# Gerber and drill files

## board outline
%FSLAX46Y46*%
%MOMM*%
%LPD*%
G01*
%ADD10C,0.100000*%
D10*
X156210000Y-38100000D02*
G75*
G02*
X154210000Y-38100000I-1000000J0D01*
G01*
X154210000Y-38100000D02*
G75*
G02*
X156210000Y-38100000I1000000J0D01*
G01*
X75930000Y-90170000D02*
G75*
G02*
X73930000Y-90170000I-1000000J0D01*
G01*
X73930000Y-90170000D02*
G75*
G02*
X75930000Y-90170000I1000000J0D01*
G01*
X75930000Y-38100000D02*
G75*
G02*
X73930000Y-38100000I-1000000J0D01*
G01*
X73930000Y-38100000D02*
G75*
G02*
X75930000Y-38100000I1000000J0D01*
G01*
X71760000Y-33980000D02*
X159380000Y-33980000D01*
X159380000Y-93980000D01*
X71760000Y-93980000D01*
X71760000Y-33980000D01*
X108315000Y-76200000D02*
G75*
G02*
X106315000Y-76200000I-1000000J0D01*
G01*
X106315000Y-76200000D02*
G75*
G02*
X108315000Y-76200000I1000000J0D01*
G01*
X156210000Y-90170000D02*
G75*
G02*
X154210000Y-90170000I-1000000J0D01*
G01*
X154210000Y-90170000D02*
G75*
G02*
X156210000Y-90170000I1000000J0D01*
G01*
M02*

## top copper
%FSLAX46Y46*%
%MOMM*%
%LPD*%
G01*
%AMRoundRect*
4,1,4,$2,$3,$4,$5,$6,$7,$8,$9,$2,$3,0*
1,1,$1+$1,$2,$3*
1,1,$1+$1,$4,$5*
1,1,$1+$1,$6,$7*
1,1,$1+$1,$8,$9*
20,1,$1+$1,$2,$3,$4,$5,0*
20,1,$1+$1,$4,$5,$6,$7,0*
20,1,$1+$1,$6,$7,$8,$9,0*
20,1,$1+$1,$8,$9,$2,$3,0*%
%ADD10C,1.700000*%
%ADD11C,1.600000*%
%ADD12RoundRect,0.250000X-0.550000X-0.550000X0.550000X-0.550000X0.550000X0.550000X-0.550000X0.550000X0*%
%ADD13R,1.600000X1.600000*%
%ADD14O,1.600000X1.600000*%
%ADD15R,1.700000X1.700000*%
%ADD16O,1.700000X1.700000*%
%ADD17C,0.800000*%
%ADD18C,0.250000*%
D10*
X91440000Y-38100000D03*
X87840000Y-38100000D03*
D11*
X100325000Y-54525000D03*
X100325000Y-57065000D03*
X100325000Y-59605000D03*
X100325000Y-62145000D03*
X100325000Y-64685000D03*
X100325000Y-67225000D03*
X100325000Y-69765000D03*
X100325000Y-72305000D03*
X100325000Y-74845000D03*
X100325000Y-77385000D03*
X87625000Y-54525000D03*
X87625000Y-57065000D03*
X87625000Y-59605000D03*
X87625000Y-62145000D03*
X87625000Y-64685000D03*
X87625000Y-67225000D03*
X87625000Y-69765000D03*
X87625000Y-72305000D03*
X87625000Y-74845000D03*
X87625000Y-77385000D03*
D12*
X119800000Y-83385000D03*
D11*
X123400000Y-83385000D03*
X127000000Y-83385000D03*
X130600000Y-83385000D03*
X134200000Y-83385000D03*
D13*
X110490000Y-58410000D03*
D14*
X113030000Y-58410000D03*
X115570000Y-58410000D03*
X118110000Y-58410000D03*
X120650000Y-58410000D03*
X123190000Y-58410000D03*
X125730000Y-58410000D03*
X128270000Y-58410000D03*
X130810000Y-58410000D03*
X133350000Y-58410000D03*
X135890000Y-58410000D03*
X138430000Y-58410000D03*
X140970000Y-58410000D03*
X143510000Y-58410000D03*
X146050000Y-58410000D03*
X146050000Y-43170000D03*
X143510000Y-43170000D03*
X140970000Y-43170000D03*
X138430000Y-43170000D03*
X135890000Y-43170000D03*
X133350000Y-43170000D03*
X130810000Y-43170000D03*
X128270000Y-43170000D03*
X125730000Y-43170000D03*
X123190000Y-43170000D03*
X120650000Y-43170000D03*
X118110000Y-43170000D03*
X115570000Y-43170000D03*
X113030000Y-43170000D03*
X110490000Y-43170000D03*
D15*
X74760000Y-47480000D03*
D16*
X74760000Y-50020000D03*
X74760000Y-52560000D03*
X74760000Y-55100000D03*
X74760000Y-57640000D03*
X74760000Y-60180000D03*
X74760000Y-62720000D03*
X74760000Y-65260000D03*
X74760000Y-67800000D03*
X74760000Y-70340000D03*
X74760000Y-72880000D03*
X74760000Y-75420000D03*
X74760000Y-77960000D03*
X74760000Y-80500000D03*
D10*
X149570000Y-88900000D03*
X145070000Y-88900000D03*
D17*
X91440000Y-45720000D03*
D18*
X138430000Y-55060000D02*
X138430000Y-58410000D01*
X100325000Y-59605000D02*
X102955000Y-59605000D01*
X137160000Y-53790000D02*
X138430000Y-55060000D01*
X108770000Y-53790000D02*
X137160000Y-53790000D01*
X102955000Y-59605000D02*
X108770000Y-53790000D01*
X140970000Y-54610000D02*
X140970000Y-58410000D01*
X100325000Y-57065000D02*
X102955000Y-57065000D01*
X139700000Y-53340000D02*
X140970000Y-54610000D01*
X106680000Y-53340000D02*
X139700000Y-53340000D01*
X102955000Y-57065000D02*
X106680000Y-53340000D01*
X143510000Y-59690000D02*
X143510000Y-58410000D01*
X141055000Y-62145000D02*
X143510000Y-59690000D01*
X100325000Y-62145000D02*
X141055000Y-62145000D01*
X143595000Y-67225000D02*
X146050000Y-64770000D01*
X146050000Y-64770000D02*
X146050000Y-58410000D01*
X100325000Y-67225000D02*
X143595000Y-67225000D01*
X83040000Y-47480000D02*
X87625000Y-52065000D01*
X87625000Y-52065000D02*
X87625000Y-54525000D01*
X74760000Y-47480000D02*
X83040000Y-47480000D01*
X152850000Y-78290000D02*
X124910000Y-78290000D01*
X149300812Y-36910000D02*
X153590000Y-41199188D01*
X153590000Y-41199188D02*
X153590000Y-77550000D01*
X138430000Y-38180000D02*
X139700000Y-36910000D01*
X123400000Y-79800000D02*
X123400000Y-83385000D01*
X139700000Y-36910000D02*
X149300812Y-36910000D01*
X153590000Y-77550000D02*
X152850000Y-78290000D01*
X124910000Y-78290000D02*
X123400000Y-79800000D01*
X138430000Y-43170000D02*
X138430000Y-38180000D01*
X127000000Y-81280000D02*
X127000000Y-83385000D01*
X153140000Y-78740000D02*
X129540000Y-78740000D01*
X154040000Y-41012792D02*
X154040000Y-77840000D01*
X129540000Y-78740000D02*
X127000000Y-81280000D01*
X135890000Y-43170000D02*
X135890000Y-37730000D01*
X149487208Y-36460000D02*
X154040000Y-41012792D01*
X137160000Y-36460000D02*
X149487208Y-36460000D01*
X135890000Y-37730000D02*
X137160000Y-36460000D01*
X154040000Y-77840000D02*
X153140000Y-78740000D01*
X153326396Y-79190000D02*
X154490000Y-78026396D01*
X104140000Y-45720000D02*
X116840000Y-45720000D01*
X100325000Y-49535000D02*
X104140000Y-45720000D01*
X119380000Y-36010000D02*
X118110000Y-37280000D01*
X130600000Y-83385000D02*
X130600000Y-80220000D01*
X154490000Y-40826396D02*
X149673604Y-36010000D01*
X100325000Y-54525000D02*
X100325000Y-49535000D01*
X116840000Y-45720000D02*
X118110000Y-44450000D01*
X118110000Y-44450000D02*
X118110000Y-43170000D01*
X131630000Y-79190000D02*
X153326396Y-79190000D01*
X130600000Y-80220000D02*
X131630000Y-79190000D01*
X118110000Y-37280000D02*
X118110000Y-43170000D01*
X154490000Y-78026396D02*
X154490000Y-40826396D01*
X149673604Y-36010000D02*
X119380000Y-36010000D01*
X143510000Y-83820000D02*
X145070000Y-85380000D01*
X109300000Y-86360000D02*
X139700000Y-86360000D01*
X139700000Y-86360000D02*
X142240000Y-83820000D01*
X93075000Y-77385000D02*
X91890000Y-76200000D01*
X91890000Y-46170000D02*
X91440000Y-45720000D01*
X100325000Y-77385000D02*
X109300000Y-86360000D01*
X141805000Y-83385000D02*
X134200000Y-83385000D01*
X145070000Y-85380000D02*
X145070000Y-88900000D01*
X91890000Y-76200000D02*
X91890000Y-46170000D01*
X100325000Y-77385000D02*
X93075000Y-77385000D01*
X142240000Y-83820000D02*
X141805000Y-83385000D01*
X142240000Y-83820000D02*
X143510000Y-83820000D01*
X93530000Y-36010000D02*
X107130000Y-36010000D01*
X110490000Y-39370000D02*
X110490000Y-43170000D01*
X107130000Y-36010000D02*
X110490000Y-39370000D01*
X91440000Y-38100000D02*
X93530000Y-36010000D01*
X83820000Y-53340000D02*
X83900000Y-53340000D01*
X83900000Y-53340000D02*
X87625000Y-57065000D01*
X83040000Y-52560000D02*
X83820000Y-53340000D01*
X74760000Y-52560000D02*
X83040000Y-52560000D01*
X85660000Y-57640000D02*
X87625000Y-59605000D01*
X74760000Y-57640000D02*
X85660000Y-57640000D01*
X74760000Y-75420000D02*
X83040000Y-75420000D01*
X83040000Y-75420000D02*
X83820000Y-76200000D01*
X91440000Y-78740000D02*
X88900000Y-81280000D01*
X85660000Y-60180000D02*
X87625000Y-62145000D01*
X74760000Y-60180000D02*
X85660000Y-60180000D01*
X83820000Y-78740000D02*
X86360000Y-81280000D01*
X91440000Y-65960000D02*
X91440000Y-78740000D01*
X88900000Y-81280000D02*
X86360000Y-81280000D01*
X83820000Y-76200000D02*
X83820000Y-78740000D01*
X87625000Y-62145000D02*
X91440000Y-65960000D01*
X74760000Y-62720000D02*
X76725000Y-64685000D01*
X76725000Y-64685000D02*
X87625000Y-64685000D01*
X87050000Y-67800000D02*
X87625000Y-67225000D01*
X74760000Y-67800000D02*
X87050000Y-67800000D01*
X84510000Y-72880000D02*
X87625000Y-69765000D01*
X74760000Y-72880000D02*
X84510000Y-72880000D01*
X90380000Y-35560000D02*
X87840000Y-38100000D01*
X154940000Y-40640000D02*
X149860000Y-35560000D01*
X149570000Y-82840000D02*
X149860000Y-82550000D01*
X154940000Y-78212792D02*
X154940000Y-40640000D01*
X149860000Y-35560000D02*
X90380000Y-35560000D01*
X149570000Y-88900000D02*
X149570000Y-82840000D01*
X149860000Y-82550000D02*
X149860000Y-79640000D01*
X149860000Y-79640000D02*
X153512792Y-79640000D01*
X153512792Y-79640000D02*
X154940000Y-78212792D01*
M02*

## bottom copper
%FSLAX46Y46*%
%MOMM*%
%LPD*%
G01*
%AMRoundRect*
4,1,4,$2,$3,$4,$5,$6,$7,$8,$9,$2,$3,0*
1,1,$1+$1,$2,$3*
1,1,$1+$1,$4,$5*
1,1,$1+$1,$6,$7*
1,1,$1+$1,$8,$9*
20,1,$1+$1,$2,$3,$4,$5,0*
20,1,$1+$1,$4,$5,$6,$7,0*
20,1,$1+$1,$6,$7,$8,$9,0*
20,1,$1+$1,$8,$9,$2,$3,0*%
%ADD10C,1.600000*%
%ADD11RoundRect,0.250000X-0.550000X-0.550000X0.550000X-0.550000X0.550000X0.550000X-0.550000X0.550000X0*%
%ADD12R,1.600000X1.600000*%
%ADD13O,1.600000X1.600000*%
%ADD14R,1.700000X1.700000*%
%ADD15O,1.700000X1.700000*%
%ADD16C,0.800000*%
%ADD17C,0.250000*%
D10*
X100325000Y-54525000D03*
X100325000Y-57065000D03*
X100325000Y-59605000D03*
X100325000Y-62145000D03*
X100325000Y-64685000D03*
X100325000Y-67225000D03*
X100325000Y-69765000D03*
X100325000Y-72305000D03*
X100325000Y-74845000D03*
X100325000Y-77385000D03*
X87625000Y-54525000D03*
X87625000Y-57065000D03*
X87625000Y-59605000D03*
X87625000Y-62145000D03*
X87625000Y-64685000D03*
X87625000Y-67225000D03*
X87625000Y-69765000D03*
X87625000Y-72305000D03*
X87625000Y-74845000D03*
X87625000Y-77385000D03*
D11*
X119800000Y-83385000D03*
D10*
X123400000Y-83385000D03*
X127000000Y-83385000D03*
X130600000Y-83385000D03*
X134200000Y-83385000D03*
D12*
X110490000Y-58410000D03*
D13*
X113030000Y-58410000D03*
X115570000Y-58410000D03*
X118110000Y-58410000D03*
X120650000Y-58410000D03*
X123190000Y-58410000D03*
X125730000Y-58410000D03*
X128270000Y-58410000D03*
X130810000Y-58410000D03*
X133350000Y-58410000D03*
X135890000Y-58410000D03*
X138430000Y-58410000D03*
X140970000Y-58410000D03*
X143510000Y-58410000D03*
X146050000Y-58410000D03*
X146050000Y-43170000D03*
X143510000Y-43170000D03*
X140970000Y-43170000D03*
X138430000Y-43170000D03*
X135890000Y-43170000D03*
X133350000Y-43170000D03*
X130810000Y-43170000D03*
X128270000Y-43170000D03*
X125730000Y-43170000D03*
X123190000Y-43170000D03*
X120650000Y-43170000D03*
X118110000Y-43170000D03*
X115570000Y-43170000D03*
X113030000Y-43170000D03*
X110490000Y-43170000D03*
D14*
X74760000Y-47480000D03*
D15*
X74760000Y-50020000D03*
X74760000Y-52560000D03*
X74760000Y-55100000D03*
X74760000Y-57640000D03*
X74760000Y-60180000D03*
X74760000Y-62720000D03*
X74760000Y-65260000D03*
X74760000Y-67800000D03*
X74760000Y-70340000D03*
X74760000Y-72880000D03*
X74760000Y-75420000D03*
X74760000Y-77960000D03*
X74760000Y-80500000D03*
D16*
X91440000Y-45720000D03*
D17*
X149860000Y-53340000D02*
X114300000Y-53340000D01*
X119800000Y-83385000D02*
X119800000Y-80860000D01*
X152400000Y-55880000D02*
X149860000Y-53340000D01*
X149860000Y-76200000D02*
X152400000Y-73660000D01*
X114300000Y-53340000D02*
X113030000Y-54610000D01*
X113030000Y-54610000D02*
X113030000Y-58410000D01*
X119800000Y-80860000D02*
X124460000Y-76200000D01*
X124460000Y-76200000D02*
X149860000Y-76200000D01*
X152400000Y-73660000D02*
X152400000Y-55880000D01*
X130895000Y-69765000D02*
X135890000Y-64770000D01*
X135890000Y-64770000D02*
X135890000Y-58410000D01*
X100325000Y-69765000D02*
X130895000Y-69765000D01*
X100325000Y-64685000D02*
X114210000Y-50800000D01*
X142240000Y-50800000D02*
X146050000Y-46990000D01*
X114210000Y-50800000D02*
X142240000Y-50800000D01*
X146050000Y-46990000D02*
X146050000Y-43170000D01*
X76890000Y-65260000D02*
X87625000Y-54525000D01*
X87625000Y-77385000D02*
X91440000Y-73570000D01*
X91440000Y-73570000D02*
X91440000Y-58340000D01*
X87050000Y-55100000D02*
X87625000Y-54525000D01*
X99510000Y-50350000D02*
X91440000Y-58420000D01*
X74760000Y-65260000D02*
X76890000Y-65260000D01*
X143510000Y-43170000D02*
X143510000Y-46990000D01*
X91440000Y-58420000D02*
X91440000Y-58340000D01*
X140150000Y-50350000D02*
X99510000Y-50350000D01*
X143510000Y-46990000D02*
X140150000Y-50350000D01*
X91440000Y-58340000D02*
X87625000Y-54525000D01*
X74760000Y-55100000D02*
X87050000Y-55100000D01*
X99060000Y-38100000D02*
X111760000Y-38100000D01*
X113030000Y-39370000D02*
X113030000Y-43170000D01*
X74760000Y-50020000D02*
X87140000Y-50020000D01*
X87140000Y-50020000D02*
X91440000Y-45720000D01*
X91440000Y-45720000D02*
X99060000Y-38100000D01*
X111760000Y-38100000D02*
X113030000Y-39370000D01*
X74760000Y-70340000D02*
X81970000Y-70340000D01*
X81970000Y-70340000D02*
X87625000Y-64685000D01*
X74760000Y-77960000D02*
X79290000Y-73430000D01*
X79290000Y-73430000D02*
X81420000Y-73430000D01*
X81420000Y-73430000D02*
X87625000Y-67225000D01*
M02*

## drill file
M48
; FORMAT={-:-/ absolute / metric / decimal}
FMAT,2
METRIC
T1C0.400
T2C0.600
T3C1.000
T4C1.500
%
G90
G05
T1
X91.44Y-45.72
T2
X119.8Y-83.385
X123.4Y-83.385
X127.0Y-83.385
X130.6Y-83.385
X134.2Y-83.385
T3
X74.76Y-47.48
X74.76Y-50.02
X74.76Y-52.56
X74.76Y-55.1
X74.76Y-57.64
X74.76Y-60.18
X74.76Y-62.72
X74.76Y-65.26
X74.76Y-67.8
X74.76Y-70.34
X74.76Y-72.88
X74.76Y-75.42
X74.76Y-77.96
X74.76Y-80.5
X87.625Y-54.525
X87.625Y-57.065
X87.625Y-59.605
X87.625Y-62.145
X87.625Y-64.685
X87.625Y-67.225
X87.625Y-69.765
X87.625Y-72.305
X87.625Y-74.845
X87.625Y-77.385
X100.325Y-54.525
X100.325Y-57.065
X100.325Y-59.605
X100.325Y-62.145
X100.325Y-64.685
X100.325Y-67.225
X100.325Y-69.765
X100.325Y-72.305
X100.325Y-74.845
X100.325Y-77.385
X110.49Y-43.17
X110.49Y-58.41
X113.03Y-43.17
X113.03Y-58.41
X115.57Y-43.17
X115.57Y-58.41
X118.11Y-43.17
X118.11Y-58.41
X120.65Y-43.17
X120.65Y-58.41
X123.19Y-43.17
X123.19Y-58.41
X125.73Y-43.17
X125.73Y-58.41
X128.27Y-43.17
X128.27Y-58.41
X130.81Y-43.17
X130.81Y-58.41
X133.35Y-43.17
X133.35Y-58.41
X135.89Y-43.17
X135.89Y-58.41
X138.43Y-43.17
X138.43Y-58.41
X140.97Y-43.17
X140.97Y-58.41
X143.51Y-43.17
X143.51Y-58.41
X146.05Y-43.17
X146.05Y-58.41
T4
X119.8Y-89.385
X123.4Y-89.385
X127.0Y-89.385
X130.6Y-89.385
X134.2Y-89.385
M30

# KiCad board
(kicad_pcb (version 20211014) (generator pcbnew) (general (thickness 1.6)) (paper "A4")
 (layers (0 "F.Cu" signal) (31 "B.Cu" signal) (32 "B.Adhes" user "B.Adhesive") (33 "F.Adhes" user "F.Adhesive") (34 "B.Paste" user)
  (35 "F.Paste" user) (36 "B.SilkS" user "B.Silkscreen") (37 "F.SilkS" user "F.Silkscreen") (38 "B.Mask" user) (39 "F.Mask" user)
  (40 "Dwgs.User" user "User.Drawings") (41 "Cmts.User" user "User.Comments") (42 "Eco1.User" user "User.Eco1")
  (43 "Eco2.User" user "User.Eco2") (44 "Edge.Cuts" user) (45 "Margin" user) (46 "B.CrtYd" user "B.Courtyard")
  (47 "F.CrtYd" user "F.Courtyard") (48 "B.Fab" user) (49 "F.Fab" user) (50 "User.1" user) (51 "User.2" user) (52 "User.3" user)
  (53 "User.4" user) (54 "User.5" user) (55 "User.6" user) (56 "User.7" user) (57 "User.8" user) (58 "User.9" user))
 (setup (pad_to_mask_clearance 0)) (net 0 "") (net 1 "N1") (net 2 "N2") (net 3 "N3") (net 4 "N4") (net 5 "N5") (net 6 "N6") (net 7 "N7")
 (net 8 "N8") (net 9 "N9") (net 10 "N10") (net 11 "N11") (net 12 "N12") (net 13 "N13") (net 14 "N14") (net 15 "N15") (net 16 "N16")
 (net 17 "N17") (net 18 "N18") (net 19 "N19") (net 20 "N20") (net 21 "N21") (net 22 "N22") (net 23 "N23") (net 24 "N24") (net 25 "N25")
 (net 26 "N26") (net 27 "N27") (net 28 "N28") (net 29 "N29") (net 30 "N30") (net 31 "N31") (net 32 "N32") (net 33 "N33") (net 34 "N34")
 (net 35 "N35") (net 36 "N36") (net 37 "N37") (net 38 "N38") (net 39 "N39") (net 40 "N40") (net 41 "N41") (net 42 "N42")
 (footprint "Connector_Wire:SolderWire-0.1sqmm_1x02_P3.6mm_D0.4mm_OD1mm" (layer "F.Cu") (at 91.44 38.1 180)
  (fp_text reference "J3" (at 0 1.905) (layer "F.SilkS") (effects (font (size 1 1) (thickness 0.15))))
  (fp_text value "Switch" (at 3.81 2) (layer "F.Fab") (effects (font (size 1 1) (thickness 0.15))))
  (pad "1" smd circle (at 0 0 180) (size 1.7 1.7) (layers "F.Cu" "F.Paste" "F.Mask") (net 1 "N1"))
  (pad "2" smd circle (at 3.6 0 180) (size 1.7 1.7) (layers "F.Cu" "F.Paste" "F.Mask") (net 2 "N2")))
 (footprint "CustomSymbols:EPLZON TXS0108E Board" (layer "F.Cu") (at 101.595 53.255 -90)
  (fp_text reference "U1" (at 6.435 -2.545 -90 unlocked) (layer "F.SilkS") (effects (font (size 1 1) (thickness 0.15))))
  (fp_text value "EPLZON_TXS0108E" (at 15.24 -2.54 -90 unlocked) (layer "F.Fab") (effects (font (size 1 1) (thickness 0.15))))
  (pad "1" thru_hole circle (at 1.27 1.27 270) (size 1.6 1.6) (drill 1) (layers *.Cu *.Mask) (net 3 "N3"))
  (pad "2" thru_hole circle (at 3.81 1.27 270) (size 1.6 1.6) (drill 1) (layers *.Cu *.Mask) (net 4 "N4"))
  (pad "3" thru_hole circle (at 6.35 1.27 270) (size 1.6 1.6) (drill 1) (layers *.Cu *.Mask) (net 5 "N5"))
  (pad "4" thru_hole circle (at 8.89 1.27 270) (size 1.6 1.6) (drill 1) (layers *.Cu *.Mask) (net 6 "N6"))
  (pad "5" thru_hole circle (at 11.43 1.27 270) (size 1.6 1.6) (drill 1) (layers *.Cu *.Mask) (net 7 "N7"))
  (pad "6" thru_hole circle (at 13.97 1.27 270) (size 1.6 1.6) (drill 1) (layers *.Cu *.Mask) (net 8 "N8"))
  (pad "7" thru_hole circle (at 16.51 1.27 270) (size 1.6 1.6) (drill 1) (layers *.Cu *.Mask) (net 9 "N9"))
  (pad "8" thru_hole circle (at 19.05 1.27 270) (size 1.6 1.6) (drill 1) (layers *.Cu *.Mask) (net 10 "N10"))
  (pad "9" thru_hole circle (at 21.59 1.27 270) (size 1.6 1.6) (drill 1) (layers *.Cu *.Mask) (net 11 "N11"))
  (pad "10" thru_hole circle (at 24.13 1.27 270) (size 1.6 1.6) (drill 1) (layers *.Cu *.Mask) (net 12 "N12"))
  (pad "11" thru_hole circle (at 1.27 13.97 270) (size 1.6 1.6) (drill 1) (layers *.Cu *.Mask) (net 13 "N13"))
  (pad "12" thru_hole circle (at 3.81 13.97 270) (size 1.6 1.6) (drill 1) (layers *.Cu *.Mask) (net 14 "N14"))
  (pad "13" thru_hole circle (at 6.35 13.97 270) (size 1.6 1.6) (drill 1) (layers *.Cu *.Mask) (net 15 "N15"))
  (pad "14" thru_hole circle (at 8.89 13.97 270) (size 1.6 1.6) (drill 1) (layers *.Cu *.Mask) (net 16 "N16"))
  (pad "15" thru_hole circle (at 11.43 13.97 270) (size 1.6 1.6) (drill 1) (layers *.Cu *.Mask) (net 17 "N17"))
  (pad "16" thru_hole circle (at 13.97 13.97 270) (size 1.6 1.6) (drill 1) (layers *.Cu *.Mask) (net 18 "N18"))
  (pad "17" thru_hole circle (at 16.51 13.97 270) (size 1.6 1.6) (drill 1) (layers *.Cu *.Mask) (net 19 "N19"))
  (pad "18" thru_hole circle (at 19.05 13.97 270) (size 1.6 1.6) (drill 1) (layers *.Cu *.Mask) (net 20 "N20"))
  (pad "19" thru_hole circle (at 21.59 13.97 270) (size 1.6 1.6) (drill 1) (layers *.Cu *.Mask) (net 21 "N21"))
  (pad "20" thru_hole circle (at 24.13 13.97 270) (size 1.6 1.6) (drill 1) (layers *.Cu *.Mask) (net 13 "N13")))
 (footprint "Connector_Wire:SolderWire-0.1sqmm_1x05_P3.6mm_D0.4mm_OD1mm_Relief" (layer "F.Cu") (at 119.8 83.385)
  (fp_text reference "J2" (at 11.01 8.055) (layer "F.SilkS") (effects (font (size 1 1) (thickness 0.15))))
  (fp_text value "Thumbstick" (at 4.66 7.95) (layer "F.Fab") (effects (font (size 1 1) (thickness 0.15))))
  (pad "" np_thru_hole circle (at 10.8 6) (size 1.5 1.5) (drill 1.5) (layers *.Cu *.Mask))
  (pad "" np_thru_hole circle (at 3.6 6) (size 1.5 1.5) (drill 1.5) (layers *.Cu *.Mask))
  (pad "" np_thru_hole circle (at 0 6) (size 1.5 1.5) (drill 1.5) (layers *.Cu *.Mask))
  (pad "" np_thru_hole circle (at 14.4 6) (size 1.5 1.5) (drill 1.5) (layers *.Cu *.Mask))
  (pad "" np_thru_hole circle (at 7.2 6) (size 1.5 1.5) (drill 1.5) (layers *.Cu *.Mask))
  (pad "1" thru_hole roundrect (at 0 0) (size 1.6 1.6) (drill 0.6) (layers *.Cu *.Mask) (roundrect_rratio 0.15625) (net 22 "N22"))
  (pad "2" thru_hole circle (at 3.6 0) (size 1.6 1.6) (drill 0.6) (layers *.Cu *.Mask) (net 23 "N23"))
  (pad "3" thru_hole circle (at 7.2 0) (size 1.6 1.6) (drill 0.6) (layers *.Cu *.Mask) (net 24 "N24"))
  (pad "4" thru_hole circle (at 10.8 0) (size 1.6 1.6) (drill 0.6) (layers *.Cu *.Mask) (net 3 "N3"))
  (pad "5" thru_hole circle (at 14.4 0) (size 1.6 1.6) (drill 0.6) (layers *.Cu *.Mask) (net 12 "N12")))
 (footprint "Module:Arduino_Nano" (layer "F.Cu") (at 110.49 58.41 90)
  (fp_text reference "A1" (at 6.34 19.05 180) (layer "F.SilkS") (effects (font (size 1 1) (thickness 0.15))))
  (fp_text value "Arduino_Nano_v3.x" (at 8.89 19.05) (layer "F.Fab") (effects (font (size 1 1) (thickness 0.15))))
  (pad "1" thru_hole rect (at 0 0 90) (size 1.6 1.6) (drill 1) (layers *.Cu *.Mask) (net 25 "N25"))
  (pad "2" thru_hole oval (at 0 2.54 90) (size 1.6 1.6) (drill 1) (layers *.Cu *.Mask) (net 22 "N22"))
  (pad "3" thru_hole oval (at 0 5.08 90) (size 1.6 1.6) (drill 1) (layers *.Cu *.Mask) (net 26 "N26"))
  (pad "4" thru_hole oval (at 0 7.62 90) (size 1.6 1.6) (drill 1) (layers *.Cu *.Mask) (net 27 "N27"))
  (pad "5" thru_hole oval (at 0 10.16 90) (size 1.6 1.6) (drill 1) (layers *.Cu *.Mask) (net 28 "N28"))
  (pad "6" thru_hole oval (at 0 12.7 90) (size 1.6 1.6) (drill 1) (layers *.Cu *.Mask) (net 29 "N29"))
  (pad "7" thru_hole oval (at 0 15.24 90) (size 1.6 1.6) (drill 1) (layers *.Cu *.Mask) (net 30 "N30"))
  (pad "8" thru_hole oval (at 0 17.78 90) (size 1.6 1.6) (drill 1) (layers *.Cu *.Mask) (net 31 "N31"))
  (pad "9" thru_hole oval (at 0 20.32 90) (size 1.6 1.6) (drill 1) (layers *.Cu *.Mask) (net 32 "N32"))
  (pad "10" thru_hole oval (at 0 22.86 90) (size 1.6 1.6) (drill 1) (layers *.Cu *.Mask) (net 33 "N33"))
  (pad "11" thru_hole oval (at 0 25.4 90) (size 1.6 1.6) (drill 1) (layers *.Cu *.Mask) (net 9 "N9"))
  (pad "12" thru_hole oval (at 0 27.94 90) (size 1.6 1.6) (drill 1) (layers *.Cu *.Mask) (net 5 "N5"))
  (pad "13" thru_hole oval (at 0 30.48 90) (size 1.6 1.6) (drill 1) (layers *.Cu *.Mask) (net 4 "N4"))
  (pad "14" thru_hole oval (at 0 33.02 90) (size 1.6 1.6) (drill 1) (layers *.Cu *.Mask) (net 6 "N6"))
  (pad "15" thru_hole oval (at 0 35.56 90) (size 1.6 1.6) (drill 1) (layers *.Cu *.Mask) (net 8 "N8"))
  (pad "16" thru_hole oval (at 15.24 35.56 90) (size 1.6 1.6) (drill 1) (layers *.Cu *.Mask) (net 7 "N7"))
  (pad "17" thru_hole oval (at 15.24 33.02 90) (size 1.6 1.6) (drill 1) (layers *.Cu *.Mask) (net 13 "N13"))
  (pad "18" thru_hole oval (at 15.24 30.48 90) (size 1.6 1.6) (drill 1) (layers *.Cu *.Mask) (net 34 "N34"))
  (pad "19" thru_hole oval (at 15.24 27.94 90) (size 1.6 1.6) (drill 1) (layers *.Cu *.Mask) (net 23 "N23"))
  (pad "20" thru_hole oval (at 15.24 25.4 90) (size 1.6 1.6) (drill 1) (layers *.Cu *.Mask) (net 24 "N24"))
  (pad "21" thru_hole oval (at 15.24 22.86 90) (size 1.6 1.6) (drill 1) (layers *.Cu *.Mask) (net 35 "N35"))
  (pad "22" thru_hole oval (at 15.24 20.32 90) (size 1.6 1.6) (drill 1) (layers *.Cu *.Mask) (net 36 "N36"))
  (pad "23" thru_hole oval (at 15.24 17.78 90) (size 1.6 1.6) (drill 1) (layers *.Cu *.Mask) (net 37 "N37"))
  (pad "24" thru_hole oval (at 15.24 15.24 90) (size 1.6 1.6) (drill 1) (layers *.Cu *.Mask) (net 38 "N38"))
  (pad "25" thru_hole oval (at 15.24 12.7 90) (size 1.6 1.6) (drill 1) (layers *.Cu *.Mask) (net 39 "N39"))
  (pad "26" thru_hole oval (at 15.24 10.16 90) (size 1.6 1.6) (drill 1) (layers *.Cu *.Mask) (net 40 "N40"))
  (pad "27" thru_hole oval (at 15.24 7.62 90) (size 1.6 1.6) (drill 1) (layers *.Cu *.Mask) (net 3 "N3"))
  (pad "28" thru_hole oval (at 15.24 5.08 90) (size 1.6 1.6) (drill 1) (layers *.Cu *.Mask) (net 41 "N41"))
  (pad "29" thru_hole oval (at 15.24 2.54 90) (size 1.6 1.6) (drill 1) (layers *.Cu *.Mask) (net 12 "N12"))
  (pad "30" thru_hole oval (at 15.24 0 90) (size 1.6 1.6) (drill 1) (layers *.Cu *.Mask) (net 1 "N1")))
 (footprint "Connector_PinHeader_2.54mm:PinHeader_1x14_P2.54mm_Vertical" (layer "F.Cu") (at 74.76 47.48)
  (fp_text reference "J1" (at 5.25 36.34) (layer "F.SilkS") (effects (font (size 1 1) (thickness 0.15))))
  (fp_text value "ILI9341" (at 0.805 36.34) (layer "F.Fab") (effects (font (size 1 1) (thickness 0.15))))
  (pad "1" thru_hole rect (at 0 0) (size 1.7 1.7) (drill 1) (layers *.Cu *.Mask) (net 13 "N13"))
  (pad "2" thru_hole oval (at 0 2.54) (size 1.7 1.7) (drill 1) (layers *.Cu *.Mask) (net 12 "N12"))
  (pad "3" thru_hole oval (at 0 5.08) (size 1.7 1.7) (drill 1) (layers *.Cu *.Mask) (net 14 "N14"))
  (pad "4" thru_hole oval (at 0 7.62) (size 1.7 1.7) (drill 1) (layers *.Cu *.Mask) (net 13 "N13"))
  (pad "5" thru_hole oval (at 0 10.16) (size 1.7 1.7) (drill 1) (layers *.Cu *.Mask) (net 15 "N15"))
  (pad "6" thru_hole oval (at 0 12.7) (size 1.7 1.7) (drill 1) (layers *.Cu *.Mask) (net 16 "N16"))
  (pad "7" thru_hole oval (at 0 15.24) (size 1.7 1.7) (drill 1) (layers *.Cu *.Mask) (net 17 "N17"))
  (pad "8" thru_hole oval (at 0 17.78) (size 1.7 1.7) (drill 1) (layers *.Cu *.Mask) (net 13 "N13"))
  (pad "9" thru_hole oval (at 0 20.32) (size 1.7 1.7) (drill 1) (layers *.Cu *.Mask) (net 18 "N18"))
  (pad "10" thru_hole oval (at 0 22.86) (size 1.7 1.7) (drill 1) (layers *.Cu *.Mask) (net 17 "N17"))
  (pad "11" thru_hole oval (at 0 25.4) (size 1.7 1.7) (drill 1) (layers *.Cu *.Mask) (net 19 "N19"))
  (pad "12" thru_hole oval (at 0 27.94) (size 1.7 1.7) (drill 1) (layers *.Cu *.Mask) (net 16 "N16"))
  (pad "13" thru_hole oval (at 0 30.48) (size 1.7 1.7) (drill 1) (layers *.Cu *.Mask) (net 18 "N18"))
  (pad "14" thru_hole oval (at 0 33.02) (size 1.7 1.7) (drill 1) (layers *.Cu *.Mask) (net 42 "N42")))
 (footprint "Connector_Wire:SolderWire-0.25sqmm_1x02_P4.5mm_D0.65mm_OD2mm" (layer "F.Cu") (at 149.57 88.9 180)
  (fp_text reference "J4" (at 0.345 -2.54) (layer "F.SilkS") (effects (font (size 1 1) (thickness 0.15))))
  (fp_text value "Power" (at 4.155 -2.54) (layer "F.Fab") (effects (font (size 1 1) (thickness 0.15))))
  (pad "1" smd circle (at 0 0 180) (size 1.7 1.7) (layers "F.Cu" "F.Paste" "F.Mask") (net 2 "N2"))
  (pad "2" smd circle (at 4.5 0 180) (size 1.7 1.7) (layers "F.Cu" "F.Paste" "F.Mask") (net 12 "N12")))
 (gr_circle (center 155.21 38.1) (end 156.21 38.1) (layer "Edge.Cuts") (width 0.1) (fill none))
 (gr_circle (center 74.93 90.17) (end 75.93 90.17) (layer "Edge.Cuts") (width 0.1) (fill none))
 (gr_circle (center 74.93 38.1) (end 75.93 38.1) (layer "Edge.Cuts") (width 0.1) (fill none))
 (gr_rect (start 71.76 33.98) (end 159.38 93.98) (layer "Edge.Cuts") (width 0.1) (fill none))
 (gr_circle (center 107.315 76.2) (end 108.315 76.2) (layer "Edge.Cuts") (width 0.1) (fill none))
 (gr_circle (center 155.21 90.17) (end 156.21 90.17) (layer "Edge.Cuts") (width 0.1) (fill none))
 (segment (start 149.86 53.34) (end 114.3 53.34) (width 0.25) (layer "B.Cu") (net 22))
 (segment (start 119.8 83.385) (end 119.8 80.86) (width 0.25) (layer "B.Cu") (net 22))
 (segment (start 152.4 55.88) (end 149.86 53.34) (width 0.25) (layer "B.Cu") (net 22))
 (segment (start 149.86 76.2) (end 152.4 73.66) (width 0.25) (layer "B.Cu") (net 22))
 (segment (start 114.3 53.34) (end 113.03 54.61) (width 0.25) (layer "B.Cu") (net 22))
 (segment (start 113.03 54.61) (end 113.03 58.41) (width 0.25) (layer "B.Cu") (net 22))
 (segment (start 119.8 80.86) (end 124.46 76.2) (width 0.25) (layer "B.Cu") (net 22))
 (segment (start 124.46 76.2) (end 149.86 76.2) (width 0.25) (layer "B.Cu") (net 22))
 (segment (start 152.4 73.66) (end 152.4 55.88) (width 0.25) (layer "B.Cu") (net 22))
 (segment (start 130.895 69.765) (end 135.89 64.77) (width 0.25) (layer "B.Cu") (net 9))
 (segment (start 135.89 64.77) (end 135.89 58.41) (width 0.25) (layer "B.Cu") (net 9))
 (segment (start 100.325 69.765) (end 130.895 69.765) (width 0.25) (layer "B.Cu") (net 9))
 (segment (start 138.43 55.06) (end 138.43 58.41) (width 0.25) (layer "F.Cu") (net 5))
 (segment (start 100.325 59.605) (end 102.955 59.605) (width 0.25) (layer "F.Cu") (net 5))
 (segment (start 137.16 53.79) (end 138.43 55.06) (width 0.25) (layer "F.Cu") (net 5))
 (segment (start 108.77 53.79) (end 137.16 53.79) (width 0.25) (layer "F.Cu") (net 5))
 (segment (start 102.955 59.605) (end 108.77 53.79) (width 0.25) (layer "F.Cu") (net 5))
 (segment (start 140.97 54.61) (end 140.97 58.41) (width 0.25) (layer "F.Cu") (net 4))
 (segment (start 100.325 57.065) (end 102.955 57.065) (width 0.25) (layer "F.Cu") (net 4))
 (segment (start 139.7 53.34) (end 140.97 54.61) (width 0.25) (layer "F.Cu") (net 4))
 (segment (start 106.68 53.34) (end 139.7 53.34) (width 0.25) (layer "F.Cu") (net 4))
 (segment (start 102.955 57.065) (end 106.68 53.34) (width 0.25) (layer "F.Cu") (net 4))
 (segment (start 143.51 59.69) (end 143.51 58.41) (width 0.25) (layer "F.Cu") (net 6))
 (segment (start 141.055 62.145) (end 143.51 59.69) (width 0.25) (layer "F.Cu") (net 6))
 (segment (start 100.325 62.145) (end 141.055 62.145) (width 0.25) (layer "F.Cu") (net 6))
 (segment (start 143.595 67.225) (end 146.05 64.77) (width 0.25) (layer "F.Cu") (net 8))
 (segment (start 146.05 64.77) (end 146.05 58.41) (width 0.25) (layer "F.Cu") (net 8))
 (segment (start 100.325 67.225) (end 143.595 67.225) (width 0.25) (layer "F.Cu") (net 8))
 (segment (start 100.325 64.685) (end 114.21 50.8) (width 0.25) (layer "B.Cu") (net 7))
 (segment (start 142.24 50.8) (end 146.05 46.99) (width 0.25) (layer "B.Cu") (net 7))
 (segment (start 114.21 50.8) (end 142.24 50.8) (width 0.25) (layer "B.Cu") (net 7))
 (segment (start 146.05 46.99) (end 146.05 43.17) (width 0.25) (layer "B.Cu") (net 7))
 (segment (start 83.04 47.48) (end 87.625 52.065) (width 0.25) (layer "F.Cu") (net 13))
 (segment (start 87.625 52.065) (end 87.625 54.525) (width 0.25) (layer "F.Cu") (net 13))
 (segment (start 74.76 47.48) (end 83.04 47.48) (width 0.25) (layer "F.Cu") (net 13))
 (segment (start 76.89 65.26) (end 87.625 54.525) (width 0.25) (layer "B.Cu") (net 13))
 (segment (start 87.625 77.385) (end 91.44 73.57) (width 0.25) (layer "B.Cu") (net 13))
 (segment (start 91.44 73.57) (end 91.44 58.34) (width 0.25) (layer "B.Cu") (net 13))
 (segment (start 87.05 55.1) (end 87.625 54.525) (width 0.25) (layer "B.Cu") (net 13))
 (segment (start 99.51 50.35) (end 91.44 58.42) (width 0.25) (layer "B.Cu") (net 13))
 (segment (start 74.76 65.26) (end 76.89 65.26) (width 0.25) (layer "B.Cu") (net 13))
 (segment (start 143.51 43.17) (end 143.51 46.99) (width 0.25) (layer "B.Cu") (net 13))
 (segment (start 91.44 58.42) (end 91.44 58.34) (width 0.25) (layer "B.Cu") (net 13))
 (segment (start 140.15 50.35) (end 99.51 50.35) (width 0.25) (layer "B.Cu") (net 13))
 (segment (start 143.51 46.99) (end 140.15 50.35) (width 0.25) (layer "B.Cu") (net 13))
 (segment (start 91.44 58.34) (end 87.625 54.525) (width 0.25) (layer "B.Cu") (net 13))
 (segment (start 74.76 55.1) (end 87.05 55.1) (width 0.25) (layer "B.Cu") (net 13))
 (segment (start 152.85 78.29) (end 124.91 78.29) (width 0.25) (layer "F.Cu") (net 23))
 (segment (start 149.300812 36.91) (end 153.59 41.199188) (width 0.25) (layer "F.Cu") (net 23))
 (segment (start 153.59 41.199188) (end 153.59 77.55) (width 0.25) (layer "F.Cu") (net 23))
 (segment (start 138.43 38.18) (end 139.7 36.91) (width 0.25) (layer "F.Cu") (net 23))
 (segment (start 123.4 79.8) (end 123.4 83.385) (width 0.25) (layer "F.Cu") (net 23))
 (segment (start 139.7 36.91) (end 149.300812 36.91) (width 0.25) (layer "F.Cu") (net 23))
 (segment (start 153.59 77.55) (end 152.85 78.29) (width 0.25) (layer "F.Cu") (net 23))
 (segment (start 124.91 78.29) (end 123.4 79.8) (width 0.25) (layer "F.Cu") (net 23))
 (segment (start 138.43 43.17) (end 138.43 38.18) (width 0.25) (layer "F.Cu") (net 23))
 (segment (start 127 81.28) (end 127 83.385) (width 0.25) (layer "F.Cu") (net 24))
 (segment (start 153.14 78.74) (end 129.54 78.74) (width 0.25) (layer "F.Cu") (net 24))
 (segment (start 154.04 41.012792) (end 154.04 77.84) (width 0.25) (layer "F.Cu") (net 24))
 (segment (start 129.54 78.74) (end 127 81.28) (width 0.25) (layer "F.Cu") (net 24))
 (segment (start 135.89 43.17) (end 135.89 37.73) (width 0.25) (layer "F.Cu") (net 24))
 (segment (start 149.487208 36.46) (end 154.04 41.012792) (width 0.25) (layer "F.Cu") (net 24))
 (segment (start 137.16 36.46) (end 149.487208 36.46) (width 0.25) (layer "F.Cu") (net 24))
 (segment (start 135.89 37.73) (end 137.16 36.46) (width 0.25) (layer "F.Cu") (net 24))
 (segment (start 154.04 77.84) (end 153.14 78.74) (width 0.25) (layer "F.Cu") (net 24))
 (segment (start 153.326396 79.19) (end 154.49 78.026396) (width 0.25) (layer "F.Cu") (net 3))
 (segment (start 104.14 45.72) (end 116.84 45.72) (width 0.25) (layer "F.Cu") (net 3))
 (segment (start 100.325 49.535) (end 104.14 45.72) (width 0.25) (layer "F.Cu") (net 3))
 (segment (start 119.38 36.01) (end 118.11 37.28) (width 0.25) (layer "F.Cu") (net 3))
 (segment (start 130.6 83.385) (end 130.6 80.22) (width 0.25) (layer "F.Cu") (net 3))
 (segment (start 154.49 40.826396) (end 149.673604 36.01) (width 0.25) (layer "F.Cu") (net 3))
 (segment (start 100.325 54.525) (end 100.325 49.535) (width 0.25) (layer "F.Cu") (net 3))
 (segment (start 116.84 45.72) (end 118.11 44.45) (width 0.25) (layer "F.Cu") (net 3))
 (segment (start 118.11 44.45) (end 118.11 43.17) (width 0.25) (layer "F.Cu") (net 3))
 (segment (start 131.63 79.19) (end 153.326396 79.19) (width 0.25) (layer "F.Cu") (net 3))
 (segment (start 130.6 80.22) (end 131.63 79.19) (width 0.25) (layer "F.Cu") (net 3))
 (segment (start 118.11 37.28) (end 118.11 43.17) (width 0.25) (layer "F.Cu") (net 3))
 (segment (start 154.49 78.026396) (end 154.49 40.826396) (width 0.25) (layer "F.Cu") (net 3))
 (segment (start 149.673604 36.01) (end 119.38 36.01) (width 0.25) (layer "F.Cu") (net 3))
 (segment (start 143.51 83.82) (end 145.07 85.38) (width 0.25) (layer "F.Cu") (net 12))
 (segment (start 109.3 86.36) (end 139.7 86.36) (width 0.25) (layer "F.Cu") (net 12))
 (segment (start 139.7 86.36) (end 142.24 83.82) (width 0.25) (layer "F.Cu") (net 12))
 (segment (start 93.075 77.385) (end 91.89 76.2) (width 0.25) (layer "F.Cu") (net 12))
 (segment (start 91.89 46.17) (end 91.44 45.72) (width 0.25) (layer "F.Cu") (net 12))
 (segment (start 100.325 77.385) (end 109.3 86.36) (width 0.25) (layer "F.Cu") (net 12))
 (segment (start 141.805 83.385) (end 134.2 83.385) (width 0.25) (layer "F.Cu") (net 12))
 (segment (start 145.07 85.38) (end 145.07 88.9) (width 0.25) (layer "F.Cu") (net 12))
 (segment (start 91.89 76.2) (end 91.89 46.17) (width 0.25) (layer "F.Cu") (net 12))
 (segment (start 100.325 77.385) (end 93.075 77.385) (width 0.25) (layer "F.Cu") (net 12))
 (segment (start 142.24 83.82) (end 141.805 83.385) (width 0.25) (layer "F.Cu") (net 12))
 (segment (start 142.24 83.82) (end 143.51 83.82) (width 0.25) (layer "F.Cu") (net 12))
 (via (at 91.44 45.72) (size 0.8) (drill 0.4) (layers "F.Cu" "B.Cu") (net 12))
 (segment (start 99.06 38.1) (end 111.76 38.1) (width 0.25) (layer "B.Cu") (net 12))
 (segment (start 113.03 39.37) (end 113.03 43.17) (width 0.25) (layer "B.Cu") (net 12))
 (segment (start 74.76 50.02) (end 87.14 50.02) (width 0.25) (layer "B.Cu") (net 12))
 (segment (start 87.14 50.02) (end 91.44 45.72) (width 0.25) (layer "B.Cu") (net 12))
 (segment (start 91.44 45.72) (end 99.06 38.1) (width 0.25) (layer "B.Cu") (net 12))
 (segment (start 111.76 38.1) (end 113.03 39.37) (width 0.25) (layer "B.Cu") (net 12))
 (segment (start 93.53 36.01) (end 107.13 36.01) (width 0.25) (layer "F.Cu") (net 1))
 (segment (start 110.49 39.37) (end 110.49 43.17) (width 0.25) (layer "F.Cu") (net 1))
 (segment (start 107.13 36.01) (end 110.49 39.37) (width 0.25) (layer "F.Cu") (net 1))
 (segment (start 91.44 38.1) (end 93.53 36.01) (width 0.25) (layer "F.Cu") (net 1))
 (segment (start 83.82 53.34) (end 83.9 53.34) (width 0.25) (layer "F.Cu") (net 14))
 (segment (start 83.9 53.34) (end 87.625 57.065) (width 0.25) (layer "F.Cu") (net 14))
 (segment (start 83.04 52.56) (end 83.82 53.34) (width 0.25) (layer "F.Cu") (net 14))
 (segment (start 74.76 52.56) (end 83.04 52.56) (width 0.25) (layer "F.Cu") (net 14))
 (segment (start 85.66 57.64) (end 87.625 59.605) (width 0.25) (layer "F.Cu") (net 15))
 (segment (start 74.76 57.64) (end 85.66 57.64) (width 0.25) (layer "F.Cu") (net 15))
 (segment (start 74.76 75.42) (end 83.04 75.42) (width 0.25) (layer "F.Cu") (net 16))
 (segment (start 83.04 75.42) (end 83.82 76.2) (width 0.25) (layer "F.Cu") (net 16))
 (segment (start 91.44 78.74) (end 88.9 81.28) (width 0.25) (layer "F.Cu") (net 16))
 (segment (start 85.66 60.18) (end 87.625 62.145) (width 0.25) (layer "F.Cu") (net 16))
 (segment (start 74.76 60.18) (end 85.66 60.18) (width 0.25) (layer "F.Cu") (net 16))
 (segment (start 83.82 78.74) (end 86.36 81.28) (width 0.25) (layer "F.Cu") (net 16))
 (segment (start 91.44 65.96) (end 91.44 78.74) (width 0.25) (layer "F.Cu") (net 16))
 (segment (start 88.9 81.28) (end 86.36 81.28) (width 0.25) (layer "F.Cu") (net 16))
 (segment (start 83.82 76.2) (end 83.82 78.74) (width 0.25) (layer "F.Cu") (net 16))
 (segment (start 87.625 62.145) (end 91.44 65.96) (width 0.25) (layer "F.Cu") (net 16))
 (segment (start 74.76 62.72) (end 76.725 64.685) (width 0.25) (layer "F.Cu") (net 17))
 (segment (start 76.725 64.685) (end 87.625 64.685) (width 0.25) (layer "F.Cu") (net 17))
 (segment (start 74.76 70.34) (end 81.97 70.34) (width 0.25) (layer "B.Cu") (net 17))
 (segment (start 81.97 70.34) (end 87.625 64.685) (width 0.25) (layer "B.Cu") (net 17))
 (segment (start 87.05 67.8) (end 87.625 67.225) (width 0.25) (layer "F.Cu") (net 18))
 (segment (start 74.76 67.8) (end 87.05 67.8) (width 0.25) (layer "F.Cu") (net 18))
 (segment (start 74.76 77.96) (end 79.29 73.43) (width 0.25) (layer "B.Cu") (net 18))
 (segment (start 79.29 73.43) (end 81.42 73.43) (width 0.25) (layer "B.Cu") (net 18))
 (segment (start 81.42 73.43) (end 87.625 67.225) (width 0.25) (layer "B.Cu") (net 18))
 (segment (start 84.51 72.88) (end 87.625 69.765) (width 0.25) (layer "F.Cu") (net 19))
 (segment (start 74.76 72.88) (end 84.51 72.88) (width 0.25) (layer "F.Cu") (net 19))
 (segment (start 90.38 35.56) (end 87.84 38.1) (width 0.25) (layer "F.Cu") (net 2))
 (segment (start 154.94 40.64) (end 149.86 35.56) (width 0.25) (layer "F.Cu") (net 2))
 (segment (start 149.57 82.84) (end 149.86 82.55) (width 0.25) (layer "F.Cu") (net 2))
 (segment (start 154.94 78.212792) (end 154.94 40.64) (width 0.25) (layer "F.Cu") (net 2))
 (segment (start 149.86 35.56) (end 90.38 35.56) (width 0.25) (layer "F.Cu") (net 2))
 (segment (start 149.57 88.9) (end 149.57 82.84) (width 0.25) (layer "F.Cu") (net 2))
 (segment (start 149.86 82.55) (end 149.86 79.64) (width 0.25) (layer "F.Cu") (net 2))
 (segment (start 149.86 79.64) (end 153.512792 79.64) (width 0.25) (layer "F.Cu") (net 2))
 (segment (start 153.512792 79.64) (end 154.94 78.212792) (width 0.25) (layer "F.Cu") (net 2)))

